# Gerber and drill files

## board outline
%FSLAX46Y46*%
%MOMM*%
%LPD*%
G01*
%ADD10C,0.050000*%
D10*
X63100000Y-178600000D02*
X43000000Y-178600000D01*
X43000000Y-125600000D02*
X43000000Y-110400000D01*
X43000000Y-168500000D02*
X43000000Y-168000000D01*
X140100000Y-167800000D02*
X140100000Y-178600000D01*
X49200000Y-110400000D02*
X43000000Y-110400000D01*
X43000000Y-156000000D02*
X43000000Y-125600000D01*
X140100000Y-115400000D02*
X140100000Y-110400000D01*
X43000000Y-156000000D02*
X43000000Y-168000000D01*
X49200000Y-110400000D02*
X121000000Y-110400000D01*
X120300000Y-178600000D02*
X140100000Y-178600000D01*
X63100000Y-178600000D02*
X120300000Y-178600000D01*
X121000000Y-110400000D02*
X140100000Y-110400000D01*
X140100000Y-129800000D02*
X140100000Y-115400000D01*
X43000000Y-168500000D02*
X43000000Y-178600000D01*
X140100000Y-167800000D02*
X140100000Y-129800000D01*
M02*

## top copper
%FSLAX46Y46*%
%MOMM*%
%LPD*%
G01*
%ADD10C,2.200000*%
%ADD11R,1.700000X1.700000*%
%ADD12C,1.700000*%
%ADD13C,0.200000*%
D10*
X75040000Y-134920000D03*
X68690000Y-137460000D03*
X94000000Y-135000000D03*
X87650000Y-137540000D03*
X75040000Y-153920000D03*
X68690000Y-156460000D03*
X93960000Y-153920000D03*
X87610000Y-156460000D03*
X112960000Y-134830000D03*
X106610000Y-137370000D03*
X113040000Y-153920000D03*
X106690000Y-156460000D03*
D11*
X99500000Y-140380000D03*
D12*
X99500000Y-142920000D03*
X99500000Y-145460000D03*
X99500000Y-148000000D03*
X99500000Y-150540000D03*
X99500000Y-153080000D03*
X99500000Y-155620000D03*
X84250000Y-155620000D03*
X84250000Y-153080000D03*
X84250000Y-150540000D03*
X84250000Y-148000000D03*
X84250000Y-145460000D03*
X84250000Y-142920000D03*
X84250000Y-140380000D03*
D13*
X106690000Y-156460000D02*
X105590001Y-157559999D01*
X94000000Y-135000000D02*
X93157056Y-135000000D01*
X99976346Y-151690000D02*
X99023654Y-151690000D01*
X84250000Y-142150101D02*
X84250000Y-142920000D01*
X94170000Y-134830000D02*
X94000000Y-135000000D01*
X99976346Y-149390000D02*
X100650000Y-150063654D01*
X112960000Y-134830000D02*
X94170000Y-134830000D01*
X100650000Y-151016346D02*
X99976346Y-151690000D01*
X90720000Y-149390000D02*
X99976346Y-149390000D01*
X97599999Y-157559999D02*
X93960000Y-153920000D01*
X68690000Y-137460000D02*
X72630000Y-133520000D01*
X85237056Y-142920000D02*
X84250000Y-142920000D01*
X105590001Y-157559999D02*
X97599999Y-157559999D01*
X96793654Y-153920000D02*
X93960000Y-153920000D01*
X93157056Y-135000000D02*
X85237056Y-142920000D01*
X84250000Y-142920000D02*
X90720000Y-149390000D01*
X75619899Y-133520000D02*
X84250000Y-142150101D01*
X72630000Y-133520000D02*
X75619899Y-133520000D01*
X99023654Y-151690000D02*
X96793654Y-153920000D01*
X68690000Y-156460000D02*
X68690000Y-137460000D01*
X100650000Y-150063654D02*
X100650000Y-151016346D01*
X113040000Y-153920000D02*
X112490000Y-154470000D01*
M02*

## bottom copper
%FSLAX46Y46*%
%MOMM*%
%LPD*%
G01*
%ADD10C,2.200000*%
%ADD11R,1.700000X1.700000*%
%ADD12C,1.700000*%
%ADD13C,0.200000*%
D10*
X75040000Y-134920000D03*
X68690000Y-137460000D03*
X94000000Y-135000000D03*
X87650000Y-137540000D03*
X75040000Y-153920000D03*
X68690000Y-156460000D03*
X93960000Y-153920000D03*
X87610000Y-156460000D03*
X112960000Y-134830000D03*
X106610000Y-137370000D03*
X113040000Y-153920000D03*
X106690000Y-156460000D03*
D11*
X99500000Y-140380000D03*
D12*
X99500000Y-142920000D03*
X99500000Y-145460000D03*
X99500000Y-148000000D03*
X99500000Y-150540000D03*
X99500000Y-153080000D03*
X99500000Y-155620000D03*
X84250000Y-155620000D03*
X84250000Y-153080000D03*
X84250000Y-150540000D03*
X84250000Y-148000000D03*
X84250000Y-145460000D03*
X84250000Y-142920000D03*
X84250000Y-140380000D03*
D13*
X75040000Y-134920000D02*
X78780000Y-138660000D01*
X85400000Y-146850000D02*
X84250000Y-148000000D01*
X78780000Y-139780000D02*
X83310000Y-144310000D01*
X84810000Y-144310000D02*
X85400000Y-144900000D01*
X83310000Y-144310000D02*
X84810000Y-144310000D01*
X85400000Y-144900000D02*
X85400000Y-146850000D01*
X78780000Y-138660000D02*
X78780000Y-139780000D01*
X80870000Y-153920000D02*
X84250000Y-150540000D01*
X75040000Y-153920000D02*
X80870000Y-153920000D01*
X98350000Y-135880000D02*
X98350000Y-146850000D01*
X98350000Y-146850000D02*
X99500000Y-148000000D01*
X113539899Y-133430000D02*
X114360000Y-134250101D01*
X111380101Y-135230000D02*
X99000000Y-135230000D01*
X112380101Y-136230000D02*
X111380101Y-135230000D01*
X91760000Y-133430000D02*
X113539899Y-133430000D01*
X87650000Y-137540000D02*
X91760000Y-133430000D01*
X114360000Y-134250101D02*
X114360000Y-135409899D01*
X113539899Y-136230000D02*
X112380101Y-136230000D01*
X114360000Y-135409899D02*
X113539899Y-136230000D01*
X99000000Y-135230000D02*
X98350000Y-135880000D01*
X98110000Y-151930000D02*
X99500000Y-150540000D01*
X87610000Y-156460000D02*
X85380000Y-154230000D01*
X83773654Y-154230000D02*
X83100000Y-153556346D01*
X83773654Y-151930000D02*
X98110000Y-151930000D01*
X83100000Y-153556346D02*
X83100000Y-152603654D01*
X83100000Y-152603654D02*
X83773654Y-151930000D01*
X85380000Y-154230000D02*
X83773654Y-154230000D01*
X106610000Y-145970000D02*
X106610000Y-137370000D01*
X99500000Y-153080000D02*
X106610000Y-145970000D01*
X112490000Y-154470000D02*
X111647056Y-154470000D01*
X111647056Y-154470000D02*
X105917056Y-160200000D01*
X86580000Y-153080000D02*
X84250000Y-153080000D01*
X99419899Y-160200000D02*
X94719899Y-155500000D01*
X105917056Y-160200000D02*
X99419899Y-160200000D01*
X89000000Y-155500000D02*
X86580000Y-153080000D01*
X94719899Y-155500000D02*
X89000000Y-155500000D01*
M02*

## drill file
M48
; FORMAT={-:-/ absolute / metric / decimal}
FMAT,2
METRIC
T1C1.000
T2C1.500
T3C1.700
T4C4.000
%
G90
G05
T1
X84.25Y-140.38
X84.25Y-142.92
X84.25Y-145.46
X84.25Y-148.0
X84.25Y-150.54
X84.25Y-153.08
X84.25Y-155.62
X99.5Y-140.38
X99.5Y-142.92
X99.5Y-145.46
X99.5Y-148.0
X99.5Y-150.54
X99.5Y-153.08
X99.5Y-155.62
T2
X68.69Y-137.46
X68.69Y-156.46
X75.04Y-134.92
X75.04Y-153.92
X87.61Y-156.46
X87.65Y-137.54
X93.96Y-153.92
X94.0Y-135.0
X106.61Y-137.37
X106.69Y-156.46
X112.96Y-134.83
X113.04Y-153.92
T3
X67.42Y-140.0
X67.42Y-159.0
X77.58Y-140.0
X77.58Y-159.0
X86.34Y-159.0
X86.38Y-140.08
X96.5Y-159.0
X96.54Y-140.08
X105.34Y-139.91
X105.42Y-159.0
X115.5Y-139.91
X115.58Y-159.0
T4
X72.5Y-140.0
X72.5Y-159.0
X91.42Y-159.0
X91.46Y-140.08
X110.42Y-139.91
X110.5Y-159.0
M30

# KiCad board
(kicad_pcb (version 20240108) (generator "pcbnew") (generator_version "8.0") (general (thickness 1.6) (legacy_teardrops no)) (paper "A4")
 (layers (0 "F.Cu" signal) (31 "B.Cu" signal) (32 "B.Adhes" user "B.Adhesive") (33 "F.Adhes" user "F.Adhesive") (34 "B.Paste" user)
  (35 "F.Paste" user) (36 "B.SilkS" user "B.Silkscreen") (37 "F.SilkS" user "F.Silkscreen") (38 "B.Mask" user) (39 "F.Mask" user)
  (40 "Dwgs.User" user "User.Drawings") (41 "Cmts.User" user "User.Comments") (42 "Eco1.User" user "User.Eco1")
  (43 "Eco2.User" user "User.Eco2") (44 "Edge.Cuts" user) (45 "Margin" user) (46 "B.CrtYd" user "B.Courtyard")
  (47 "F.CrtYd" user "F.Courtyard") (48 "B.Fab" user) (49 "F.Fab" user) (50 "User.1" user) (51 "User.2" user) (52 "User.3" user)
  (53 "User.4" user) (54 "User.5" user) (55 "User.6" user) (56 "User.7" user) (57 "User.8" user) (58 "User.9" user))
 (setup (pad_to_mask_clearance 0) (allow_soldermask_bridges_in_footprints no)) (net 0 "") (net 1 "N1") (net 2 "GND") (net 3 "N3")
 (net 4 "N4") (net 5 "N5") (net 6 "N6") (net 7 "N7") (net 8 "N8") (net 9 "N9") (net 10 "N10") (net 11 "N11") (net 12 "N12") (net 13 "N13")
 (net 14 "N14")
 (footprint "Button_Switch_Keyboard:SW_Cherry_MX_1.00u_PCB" (layer "F.Cu") (at 75.04 134.92)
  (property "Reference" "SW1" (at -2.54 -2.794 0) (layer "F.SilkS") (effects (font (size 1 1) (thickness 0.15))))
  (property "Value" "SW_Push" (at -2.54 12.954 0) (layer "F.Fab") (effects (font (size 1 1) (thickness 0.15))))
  (pad "" np_thru_hole circle (at -7.62 5.08) (size 1.7 1.7) (drill 1.7) (layers "*.Cu" "*.Mask"))
  (pad "" np_thru_hole circle (at -2.54 5.08) (size 4 4) (drill 4) (layers "*.Cu" "*.Mask"))
  (pad "" np_thru_hole circle (at 2.54 5.08) (size 1.7 1.7) (drill 1.7) (layers "*.Cu" "*.Mask"))
  (pad "1" thru_hole circle (at 0 0) (size 2.2 2.2) (drill 1.5) (layers "*.Cu" "*.Mask") (remove_unused_layers no) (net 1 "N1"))
  (pad "2" thru_hole circle (at -6.35 2.54) (size 2.2 2.2) (drill 1.5) (layers "*.Cu" "*.Mask") (remove_unused_layers no) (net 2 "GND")))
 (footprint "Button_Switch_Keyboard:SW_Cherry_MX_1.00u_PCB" (layer "F.Cu") (at 94 135)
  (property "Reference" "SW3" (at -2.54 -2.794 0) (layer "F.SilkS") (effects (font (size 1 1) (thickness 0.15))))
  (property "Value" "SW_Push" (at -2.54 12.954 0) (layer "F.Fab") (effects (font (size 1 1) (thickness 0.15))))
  (pad "" np_thru_hole circle (at -7.62 5.08) (size 1.7 1.7) (drill 1.7) (layers "*.Cu" "*.Mask"))
  (pad "" np_thru_hole circle (at -2.54 5.08) (size 4 4) (drill 4) (layers "*.Cu" "*.Mask"))
  (pad "" np_thru_hole circle (at 2.54 5.08) (size 1.7 1.7) (drill 1.7) (layers "*.Cu" "*.Mask"))
  (pad "1" thru_hole circle (at 0 0) (size 2.2 2.2) (drill 1.5) (layers "*.Cu" "*.Mask") (remove_unused_layers no) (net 2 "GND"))
  (pad "2" thru_hole circle (at -6.35 2.54) (size 2.2 2.2) (drill 1.5) (layers "*.Cu" "*.Mask") (remove_unused_layers no) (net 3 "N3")))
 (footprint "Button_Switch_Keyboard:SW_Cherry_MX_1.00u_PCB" (layer "F.Cu") (at 75.04 153.92)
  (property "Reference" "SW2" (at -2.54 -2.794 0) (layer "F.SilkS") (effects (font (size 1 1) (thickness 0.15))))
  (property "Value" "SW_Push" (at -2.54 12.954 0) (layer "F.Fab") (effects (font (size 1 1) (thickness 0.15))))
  (pad "" np_thru_hole circle (at -7.62 5.08) (size 1.7 1.7) (drill 1.7) (layers "*.Cu" "*.Mask"))
  (pad "" np_thru_hole circle (at -2.54 5.08) (size 4 4) (drill 4) (layers "*.Cu" "*.Mask"))
  (pad "" np_thru_hole circle (at 2.54 5.08) (size 1.7 1.7) (drill 1.7) (layers "*.Cu" "*.Mask"))
  (pad "1" thru_hole circle (at 0 0) (size 2.2 2.2) (drill 1.5) (layers "*.Cu" "*.Mask") (remove_unused_layers no) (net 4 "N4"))
  (pad "2" thru_hole circle (at -6.35 2.54) (size 2.2 2.2) (drill 1.5) (layers "*.Cu" "*.Mask") (remove_unused_layers no) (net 2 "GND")))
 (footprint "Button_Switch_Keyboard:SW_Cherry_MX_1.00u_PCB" (layer "F.Cu") (at 93.96 153.92)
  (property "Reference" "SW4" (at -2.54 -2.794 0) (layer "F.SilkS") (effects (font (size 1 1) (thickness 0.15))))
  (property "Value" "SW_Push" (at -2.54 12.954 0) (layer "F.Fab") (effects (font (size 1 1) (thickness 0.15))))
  (pad "" np_thru_hole circle (at -7.62 5.08) (size 1.7 1.7) (drill 1.7) (layers "*.Cu" "*.Mask"))
  (pad "" np_thru_hole circle (at -2.54 5.08) (size 4 4) (drill 4) (layers "*.Cu" "*.Mask"))
  (pad "" np_thru_hole circle (at 2.54 5.08) (size 1.7 1.7) (drill 1.7) (layers "*.Cu" "*.Mask"))
  (pad "1" thru_hole circle (at 0 0) (size 2.2 2.2) (drill 1.5) (layers "*.Cu" "*.Mask") (remove_unused_layers no) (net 2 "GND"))
  (pad "2" thru_hole circle (at -6.35 2.54) (size 2.2 2.2) (drill 1.5) (layers "*.Cu" "*.Mask") (remove_unused_layers no) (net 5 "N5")))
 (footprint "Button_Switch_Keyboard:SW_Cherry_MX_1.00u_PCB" (layer "F.Cu") (at 112.96 134.83)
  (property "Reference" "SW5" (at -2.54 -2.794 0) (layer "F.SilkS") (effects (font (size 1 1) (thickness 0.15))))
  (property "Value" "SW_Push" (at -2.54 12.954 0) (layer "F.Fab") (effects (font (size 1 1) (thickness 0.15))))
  (pad "" np_thru_hole circle (at -7.62 5.08) (size 1.7 1.7) (drill 1.7) (layers "*.Cu" "*.Mask"))
  (pad "" np_thru_hole circle (at -2.54 5.08) (size 4 4) (drill 4) (layers "*.Cu" "*.Mask"))
  (pad "" np_thru_hole circle (at 2.54 5.08) (size 1.7 1.7) (drill 1.7) (layers "*.Cu" "*.Mask"))
  (pad "1" thru_hole circle (at 0 0) (size 2.2 2.2) (drill 1.5) (layers "*.Cu" "*.Mask") (remove_unused_layers no) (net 2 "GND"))
  (pad "2" thru_hole circle (at -6.35 2.54) (size 2.2 2.2) (drill 1.5) (layers "*.Cu" "*.Mask") (remove_unused_layers no) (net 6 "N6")))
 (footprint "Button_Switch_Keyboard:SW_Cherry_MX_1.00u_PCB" (layer "F.Cu") (at 113.04 153.92)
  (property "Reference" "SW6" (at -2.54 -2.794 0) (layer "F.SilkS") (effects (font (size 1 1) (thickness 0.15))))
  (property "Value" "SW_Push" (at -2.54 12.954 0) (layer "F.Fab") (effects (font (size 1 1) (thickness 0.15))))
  (pad "" np_thru_hole circle (at -7.62 5.08) (size 1.7 1.7) (drill 1.7) (layers "*.Cu" "*.Mask"))
  (pad "" np_thru_hole circle (at -2.54 5.08) (size 4 4) (drill 4) (layers "*.Cu" "*.Mask"))
  (pad "" np_thru_hole circle (at 2.54 5.08) (size 1.7 1.7) (drill 1.7) (layers "*.Cu" "*.Mask"))
  (pad "1" thru_hole circle (at 0 0) (size 2.2 2.2) (drill 1.5) (layers "*.Cu" "*.Mask") (remove_unused_layers no) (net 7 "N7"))
  (pad "2" thru_hole circle (at -6.35 2.54) (size 2.2 2.2) (drill 1.5) (layers "*.Cu" "*.Mask") (remove_unused_layers no) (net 2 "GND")))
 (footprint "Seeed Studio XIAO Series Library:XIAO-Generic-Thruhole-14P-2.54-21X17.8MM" (layer "B.Cu") (at 91.875 148 180)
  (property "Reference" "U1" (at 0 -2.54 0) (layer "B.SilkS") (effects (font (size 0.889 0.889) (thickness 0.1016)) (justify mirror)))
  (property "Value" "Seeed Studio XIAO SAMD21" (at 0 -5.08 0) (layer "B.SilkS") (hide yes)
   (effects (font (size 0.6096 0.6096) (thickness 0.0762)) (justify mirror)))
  (pad "1" thru_hole rect (at -7.625 7.62 180) (size 1.7 1.7) (drill 1) (layers "*.Cu" "*.Mask") (remove_unused_layers no) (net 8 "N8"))
  (pad "2" thru_hole circle (at -7.625 5.08 180) (size 1.7 1.7) (drill 1) (layers "*.Cu" "*.Mask") (remove_unused_layers no) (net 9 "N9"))
  (pad "3" thru_hole circle (at -7.625 2.54 180) (size 1.7 1.7) (drill 1) (layers "*.Cu" "*.Mask") (remove_unused_layers no) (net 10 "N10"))
  (pad "4" thru_hole circle (at -7.625 0 180) (size 1.7 1.7) (drill 1) (layers "*.Cu" "*.Mask") (remove_unused_layers no) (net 3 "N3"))
  (pad "5" thru_hole circle (at -7.625 -2.54 180) (size 1.7 1.7) (drill 1) (layers "*.Cu" "*.Mask") (remove_unused_layers no) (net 5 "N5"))
  (pad "6" thru_hole circle (at -7.625 -5.08) (size 1.7 1.7) (drill 1) (layers "*.Cu" "*.Mask") (remove_unused_layers no) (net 6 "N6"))
  (pad "7" thru_hole circle (at -7.625 -7.62 180) (size 1.7 1.7) (drill 1) (layers "*.Cu" "*.Mask") (remove_unused_layers no) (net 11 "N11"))
  (pad "8" thru_hole circle (at 7.625 -7.62 180) (size 1.7 1.7) (drill 1) (layers "*.Cu" "*.Mask") (remove_unused_layers no) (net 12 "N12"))
  (pad "9" thru_hole circle (at 7.625 -5.08 180) (size 1.7 1.7) (drill 1) (layers "*.Cu" "*.Mask") (remove_unused_layers no) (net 7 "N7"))
  (pad "10" thru_hole circle (at 7.625 -2.54 180) (size 1.7 1.7) (drill 1) (layers "*.Cu" "*.Mask") (remove_unused_layers no) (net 4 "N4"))
  (pad "11" thru_hole circle (at 7.625 0 180) (size 1.7 1.7) (drill 1) (layers "*.Cu" "*.Mask") (remove_unused_layers no) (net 1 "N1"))
  (pad "12" thru_hole circle (at 7.625 2.54 180) (size 1.7 1.7) (drill 1) (layers "*.Cu" "*.Mask") (remove_unused_layers no) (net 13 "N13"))
  (pad "13" thru_hole circle (at 7.625 5.08 180) (size 1.7 1.7) (drill 1) (layers "*.Cu" "*.Mask") (remove_unused_layers no) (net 2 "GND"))
  (pad "14" thru_hole circle (at 7.625 7.62 180) (size 1.7 1.7) (drill 1) (layers "*.Cu" "*.Mask") (remove_unused_layers no) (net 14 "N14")))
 (gr_line (start 63.1 178.6) (end 43 178.6) (stroke (width 0.05) (type default)) (layer "Edge.Cuts"))
 (gr_line (start 43 125.6) (end 43 110.4) (stroke (width 0.05) (type default)) (layer "Edge.Cuts"))
 (gr_line (start 43 168.5) (end 43 168) (stroke (width 0.05) (type default)) (layer "Edge.Cuts"))
 (gr_line (start 140.1 167.8) (end 140.1 178.6) (stroke (width 0.05) (type default)) (layer "Edge.Cuts"))
 (gr_line (start 49.2 110.4) (end 43 110.4) (stroke (width 0.05) (type default)) (layer "Edge.Cuts"))
 (gr_line (start 43 156) (end 43 125.6) (stroke (width 0.05) (type default)) (layer "Edge.Cuts"))
 (gr_line (start 140.1 115.4) (end 140.1 110.4) (stroke (width 0.05) (type default)) (layer "Edge.Cuts"))
 (gr_line (start 43 156) (end 43 168) (stroke (width 0.05) (type default)) (layer "Edge.Cuts"))
 (gr_line (start 49.2 110.4) (end 121 110.4) (stroke (width 0.05) (type default)) (layer "Edge.Cuts"))
 (gr_line (start 120.3 178.6) (end 140.1 178.6) (stroke (width 0.05) (type default)) (layer "Edge.Cuts"))
 (gr_line (start 63.1 178.6) (end 120.3 178.6) (stroke (width 0.05) (type default)) (layer "Edge.Cuts"))
 (gr_line (start 121 110.4) (end 140.1 110.4) (stroke (width 0.05) (type default)) (layer "Edge.Cuts"))
 (gr_line (start 140.1 129.8) (end 140.1 115.4) (stroke (width 0.05) (type default)) (layer "Edge.Cuts"))
 (gr_line (start 43 168.5) (end 43 178.6) (stroke (width 0.05) (type default)) (layer "Edge.Cuts"))
 (gr_line (start 140.1 167.8) (end 140.1 129.8) (stroke (width 0.05) (type default)) (layer "Edge.Cuts"))
 (segment (start 106.69 156.46) (end 105.590001 157.559999) (width 0.2) (layer "F.Cu") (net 2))
 (segment (start 94 135) (end 93.157056 135) (width 0.2) (layer "F.Cu") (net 2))
 (segment (start 99.976346 151.69) (end 99.023654 151.69) (width 0.2) (layer "F.Cu") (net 2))
 (segment (start 84.25 142.150101) (end 84.25 142.92) (width 0.2) (layer "F.Cu") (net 2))
 (segment (start 94.17 134.83) (end 94 135) (width 0.2) (layer "F.Cu") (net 2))
 (segment (start 99.976346 149.39) (end 100.65 150.063654) (width 0.2) (layer "F.Cu") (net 2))
 (segment (start 112.96 134.83) (end 94.17 134.83) (width 0.2) (layer "F.Cu") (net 2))
 (segment (start 100.65 151.016346) (end 99.976346 151.69) (width 0.2) (layer "F.Cu") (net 2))
 (segment (start 90.72 149.39) (end 99.976346 149.39) (width 0.2) (layer "F.Cu") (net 2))
 (segment (start 97.599999 157.559999) (end 93.96 153.92) (width 0.2) (layer "F.Cu") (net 2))
 (segment (start 68.69 137.46) (end 72.63 133.52) (width 0.2) (layer "F.Cu") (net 2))
 (segment (start 85.237056 142.92) (end 84.25 142.92) (width 0.2) (layer "F.Cu") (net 2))
 (segment (start 105.590001 157.559999) (end 97.599999 157.559999) (width 0.2) (layer "F.Cu") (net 2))
 (segment (start 96.793654 153.92) (end 93.96 153.92) (width 0.2) (layer "F.Cu") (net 2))
 (segment (start 93.157056 135) (end 85.237056 142.92) (width 0.2) (layer "F.Cu") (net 2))
 (segment (start 84.25 142.92) (end 90.72 149.39) (width 0.2) (layer "F.Cu") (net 2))
 (segment (start 75.619899 133.52) (end 84.25 142.150101) (width 0.2) (layer "F.Cu") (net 2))
 (segment (start 72.63 133.52) (end 75.619899 133.52) (width 0.2) (layer "F.Cu") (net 2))
 (segment (start 99.023654 151.69) (end 96.793654 153.92) (width 0.2) (layer "F.Cu") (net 2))
 (segment (start 68.69 156.46) (end 68.69 137.46) (width 0.2) (layer "F.Cu") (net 2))
 (segment (start 100.65 150.063654) (end 100.65 151.016346) (width 0.2) (layer "F.Cu") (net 2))
 (segment (start 75.04 134.92) (end 78.78 138.66) (width 0.2) (layer "B.Cu") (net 1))
 (segment (start 85.4 146.85) (end 84.25 148) (width 0.2) (layer "B.Cu") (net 1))
 (segment (start 78.78 139.78) (end 83.31 144.31) (width 0.2) (layer "B.Cu") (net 1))
 (segment (start 84.81 144.31) (end 85.4 144.9) (width 0.2) (layer "B.Cu") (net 1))
 (segment (start 83.31 144.31) (end 84.81 144.31) (width 0.2) (layer "B.Cu") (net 1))
 (segment (start 85.4 144.9) (end 85.4 146.85) (width 0.2) (layer "B.Cu") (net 1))
 (segment (start 78.78 138.66) (end 78.78 139.78) (width 0.2) (layer "B.Cu") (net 1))
 (segment (start 80.87 153.92) (end 84.25 150.54) (width 0.2) (layer "B.Cu") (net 4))
 (segment (start 75.04 153.92) (end 80.87 153.92) (width 0.2) (layer "B.Cu") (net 4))
 (segment (start 98.35 135.88) (end 98.35 146.85) (width 0.2) (layer "B.Cu") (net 3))
 (segment (start 98.35 146.85) (end 99.5 148) (width 0.2) (layer "B.Cu") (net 3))
 (segment (start 113.539899 133.43) (end 114.36 134.250101) (width 0.2) (layer "B.Cu") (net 3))
 (segment (start 111.380101 135.23) (end 99 135.23) (width 0.2) (layer "B.Cu") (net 3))
 (segment (start 112.380101 136.23) (end 111.380101 135.23) (width 0.2) (layer "B.Cu") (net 3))
 (segment (start 91.76 133.43) (end 113.539899 133.43) (width 0.2) (layer "B.Cu") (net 3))
 (segment (start 87.65 137.54) (end 91.76 133.43) (width 0.2) (layer "B.Cu") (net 3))
 (segment (start 114.36 134.250101) (end 114.36 135.409899) (width 0.2) (layer "B.Cu") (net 3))
 (segment (start 113.539899 136.23) (end 112.380101 136.23) (width 0.2) (layer "B.Cu") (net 3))
 (segment (start 114.36 135.409899) (end 113.539899 136.23) (width 0.2) (layer "B.Cu") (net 3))
 (segment (start 99 135.23) (end 98.35 135.88) (width 0.2) (layer "B.Cu") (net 3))
 (segment (start 98.11 151.93) (end 99.5 150.54) (width 0.2) (layer "B.Cu") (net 5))
 (segment (start 87.61 156.46) (end 85.38 154.23) (width 0.2) (layer "B.Cu") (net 5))
 (segment (start 83.773654 154.23) (end 83.1 153.556346) (width 0.2) (layer "B.Cu") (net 5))
 (segment (start 83.773654 151.93) (end 98.11 151.93) (width 0.2) (layer "B.Cu") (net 5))
 (segment (start 83.1 153.556346) (end 83.1 152.603654) (width 0.2) (layer "B.Cu") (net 5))
 (segment (start 83.1 152.603654) (end 83.773654 151.93) (width 0.2) (layer "B.Cu") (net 5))
 (segment (start 85.38 154.23) (end 83.773654 154.23) (width 0.2) (layer "B.Cu") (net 5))
 (segment (start 106.61 145.97) (end 106.61 137.37) (width 0.2) (layer "B.Cu") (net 6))
 (segment (start 99.5 153.08) (end 106.61 145.97) (width 0.2) (layer "B.Cu") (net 6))
 (segment (start 113.04 153.92) (end 112.49 154.47) (width 0.2) (layer "F.Cu") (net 7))
 (segment (start 112.49 154.47) (end 111.647056 154.47) (width 0.2) (layer "B.Cu") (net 7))
 (segment (start 111.647056 154.47) (end 105.917056 160.2) (width 0.2) (layer "B.Cu") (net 7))
 (segment (start 86.58 153.08) (end 84.25 153.08) (width 0.2) (layer "B.Cu") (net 7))
 (segment (start 99.419899 160.2) (end 94.719899 155.5) (width 0.2) (layer "B.Cu") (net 7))
 (segment (start 105.917056 160.2) (end 99.419899 160.2) (width 0.2) (layer "B.Cu") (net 7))
 (segment (start 89 155.5) (end 86.58 153.08) (width 0.2) (layer "B.Cu") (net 7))
 (segment (start 94.719899 155.5) (end 89 155.5) (width 0.2) (layer "B.Cu") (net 7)))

